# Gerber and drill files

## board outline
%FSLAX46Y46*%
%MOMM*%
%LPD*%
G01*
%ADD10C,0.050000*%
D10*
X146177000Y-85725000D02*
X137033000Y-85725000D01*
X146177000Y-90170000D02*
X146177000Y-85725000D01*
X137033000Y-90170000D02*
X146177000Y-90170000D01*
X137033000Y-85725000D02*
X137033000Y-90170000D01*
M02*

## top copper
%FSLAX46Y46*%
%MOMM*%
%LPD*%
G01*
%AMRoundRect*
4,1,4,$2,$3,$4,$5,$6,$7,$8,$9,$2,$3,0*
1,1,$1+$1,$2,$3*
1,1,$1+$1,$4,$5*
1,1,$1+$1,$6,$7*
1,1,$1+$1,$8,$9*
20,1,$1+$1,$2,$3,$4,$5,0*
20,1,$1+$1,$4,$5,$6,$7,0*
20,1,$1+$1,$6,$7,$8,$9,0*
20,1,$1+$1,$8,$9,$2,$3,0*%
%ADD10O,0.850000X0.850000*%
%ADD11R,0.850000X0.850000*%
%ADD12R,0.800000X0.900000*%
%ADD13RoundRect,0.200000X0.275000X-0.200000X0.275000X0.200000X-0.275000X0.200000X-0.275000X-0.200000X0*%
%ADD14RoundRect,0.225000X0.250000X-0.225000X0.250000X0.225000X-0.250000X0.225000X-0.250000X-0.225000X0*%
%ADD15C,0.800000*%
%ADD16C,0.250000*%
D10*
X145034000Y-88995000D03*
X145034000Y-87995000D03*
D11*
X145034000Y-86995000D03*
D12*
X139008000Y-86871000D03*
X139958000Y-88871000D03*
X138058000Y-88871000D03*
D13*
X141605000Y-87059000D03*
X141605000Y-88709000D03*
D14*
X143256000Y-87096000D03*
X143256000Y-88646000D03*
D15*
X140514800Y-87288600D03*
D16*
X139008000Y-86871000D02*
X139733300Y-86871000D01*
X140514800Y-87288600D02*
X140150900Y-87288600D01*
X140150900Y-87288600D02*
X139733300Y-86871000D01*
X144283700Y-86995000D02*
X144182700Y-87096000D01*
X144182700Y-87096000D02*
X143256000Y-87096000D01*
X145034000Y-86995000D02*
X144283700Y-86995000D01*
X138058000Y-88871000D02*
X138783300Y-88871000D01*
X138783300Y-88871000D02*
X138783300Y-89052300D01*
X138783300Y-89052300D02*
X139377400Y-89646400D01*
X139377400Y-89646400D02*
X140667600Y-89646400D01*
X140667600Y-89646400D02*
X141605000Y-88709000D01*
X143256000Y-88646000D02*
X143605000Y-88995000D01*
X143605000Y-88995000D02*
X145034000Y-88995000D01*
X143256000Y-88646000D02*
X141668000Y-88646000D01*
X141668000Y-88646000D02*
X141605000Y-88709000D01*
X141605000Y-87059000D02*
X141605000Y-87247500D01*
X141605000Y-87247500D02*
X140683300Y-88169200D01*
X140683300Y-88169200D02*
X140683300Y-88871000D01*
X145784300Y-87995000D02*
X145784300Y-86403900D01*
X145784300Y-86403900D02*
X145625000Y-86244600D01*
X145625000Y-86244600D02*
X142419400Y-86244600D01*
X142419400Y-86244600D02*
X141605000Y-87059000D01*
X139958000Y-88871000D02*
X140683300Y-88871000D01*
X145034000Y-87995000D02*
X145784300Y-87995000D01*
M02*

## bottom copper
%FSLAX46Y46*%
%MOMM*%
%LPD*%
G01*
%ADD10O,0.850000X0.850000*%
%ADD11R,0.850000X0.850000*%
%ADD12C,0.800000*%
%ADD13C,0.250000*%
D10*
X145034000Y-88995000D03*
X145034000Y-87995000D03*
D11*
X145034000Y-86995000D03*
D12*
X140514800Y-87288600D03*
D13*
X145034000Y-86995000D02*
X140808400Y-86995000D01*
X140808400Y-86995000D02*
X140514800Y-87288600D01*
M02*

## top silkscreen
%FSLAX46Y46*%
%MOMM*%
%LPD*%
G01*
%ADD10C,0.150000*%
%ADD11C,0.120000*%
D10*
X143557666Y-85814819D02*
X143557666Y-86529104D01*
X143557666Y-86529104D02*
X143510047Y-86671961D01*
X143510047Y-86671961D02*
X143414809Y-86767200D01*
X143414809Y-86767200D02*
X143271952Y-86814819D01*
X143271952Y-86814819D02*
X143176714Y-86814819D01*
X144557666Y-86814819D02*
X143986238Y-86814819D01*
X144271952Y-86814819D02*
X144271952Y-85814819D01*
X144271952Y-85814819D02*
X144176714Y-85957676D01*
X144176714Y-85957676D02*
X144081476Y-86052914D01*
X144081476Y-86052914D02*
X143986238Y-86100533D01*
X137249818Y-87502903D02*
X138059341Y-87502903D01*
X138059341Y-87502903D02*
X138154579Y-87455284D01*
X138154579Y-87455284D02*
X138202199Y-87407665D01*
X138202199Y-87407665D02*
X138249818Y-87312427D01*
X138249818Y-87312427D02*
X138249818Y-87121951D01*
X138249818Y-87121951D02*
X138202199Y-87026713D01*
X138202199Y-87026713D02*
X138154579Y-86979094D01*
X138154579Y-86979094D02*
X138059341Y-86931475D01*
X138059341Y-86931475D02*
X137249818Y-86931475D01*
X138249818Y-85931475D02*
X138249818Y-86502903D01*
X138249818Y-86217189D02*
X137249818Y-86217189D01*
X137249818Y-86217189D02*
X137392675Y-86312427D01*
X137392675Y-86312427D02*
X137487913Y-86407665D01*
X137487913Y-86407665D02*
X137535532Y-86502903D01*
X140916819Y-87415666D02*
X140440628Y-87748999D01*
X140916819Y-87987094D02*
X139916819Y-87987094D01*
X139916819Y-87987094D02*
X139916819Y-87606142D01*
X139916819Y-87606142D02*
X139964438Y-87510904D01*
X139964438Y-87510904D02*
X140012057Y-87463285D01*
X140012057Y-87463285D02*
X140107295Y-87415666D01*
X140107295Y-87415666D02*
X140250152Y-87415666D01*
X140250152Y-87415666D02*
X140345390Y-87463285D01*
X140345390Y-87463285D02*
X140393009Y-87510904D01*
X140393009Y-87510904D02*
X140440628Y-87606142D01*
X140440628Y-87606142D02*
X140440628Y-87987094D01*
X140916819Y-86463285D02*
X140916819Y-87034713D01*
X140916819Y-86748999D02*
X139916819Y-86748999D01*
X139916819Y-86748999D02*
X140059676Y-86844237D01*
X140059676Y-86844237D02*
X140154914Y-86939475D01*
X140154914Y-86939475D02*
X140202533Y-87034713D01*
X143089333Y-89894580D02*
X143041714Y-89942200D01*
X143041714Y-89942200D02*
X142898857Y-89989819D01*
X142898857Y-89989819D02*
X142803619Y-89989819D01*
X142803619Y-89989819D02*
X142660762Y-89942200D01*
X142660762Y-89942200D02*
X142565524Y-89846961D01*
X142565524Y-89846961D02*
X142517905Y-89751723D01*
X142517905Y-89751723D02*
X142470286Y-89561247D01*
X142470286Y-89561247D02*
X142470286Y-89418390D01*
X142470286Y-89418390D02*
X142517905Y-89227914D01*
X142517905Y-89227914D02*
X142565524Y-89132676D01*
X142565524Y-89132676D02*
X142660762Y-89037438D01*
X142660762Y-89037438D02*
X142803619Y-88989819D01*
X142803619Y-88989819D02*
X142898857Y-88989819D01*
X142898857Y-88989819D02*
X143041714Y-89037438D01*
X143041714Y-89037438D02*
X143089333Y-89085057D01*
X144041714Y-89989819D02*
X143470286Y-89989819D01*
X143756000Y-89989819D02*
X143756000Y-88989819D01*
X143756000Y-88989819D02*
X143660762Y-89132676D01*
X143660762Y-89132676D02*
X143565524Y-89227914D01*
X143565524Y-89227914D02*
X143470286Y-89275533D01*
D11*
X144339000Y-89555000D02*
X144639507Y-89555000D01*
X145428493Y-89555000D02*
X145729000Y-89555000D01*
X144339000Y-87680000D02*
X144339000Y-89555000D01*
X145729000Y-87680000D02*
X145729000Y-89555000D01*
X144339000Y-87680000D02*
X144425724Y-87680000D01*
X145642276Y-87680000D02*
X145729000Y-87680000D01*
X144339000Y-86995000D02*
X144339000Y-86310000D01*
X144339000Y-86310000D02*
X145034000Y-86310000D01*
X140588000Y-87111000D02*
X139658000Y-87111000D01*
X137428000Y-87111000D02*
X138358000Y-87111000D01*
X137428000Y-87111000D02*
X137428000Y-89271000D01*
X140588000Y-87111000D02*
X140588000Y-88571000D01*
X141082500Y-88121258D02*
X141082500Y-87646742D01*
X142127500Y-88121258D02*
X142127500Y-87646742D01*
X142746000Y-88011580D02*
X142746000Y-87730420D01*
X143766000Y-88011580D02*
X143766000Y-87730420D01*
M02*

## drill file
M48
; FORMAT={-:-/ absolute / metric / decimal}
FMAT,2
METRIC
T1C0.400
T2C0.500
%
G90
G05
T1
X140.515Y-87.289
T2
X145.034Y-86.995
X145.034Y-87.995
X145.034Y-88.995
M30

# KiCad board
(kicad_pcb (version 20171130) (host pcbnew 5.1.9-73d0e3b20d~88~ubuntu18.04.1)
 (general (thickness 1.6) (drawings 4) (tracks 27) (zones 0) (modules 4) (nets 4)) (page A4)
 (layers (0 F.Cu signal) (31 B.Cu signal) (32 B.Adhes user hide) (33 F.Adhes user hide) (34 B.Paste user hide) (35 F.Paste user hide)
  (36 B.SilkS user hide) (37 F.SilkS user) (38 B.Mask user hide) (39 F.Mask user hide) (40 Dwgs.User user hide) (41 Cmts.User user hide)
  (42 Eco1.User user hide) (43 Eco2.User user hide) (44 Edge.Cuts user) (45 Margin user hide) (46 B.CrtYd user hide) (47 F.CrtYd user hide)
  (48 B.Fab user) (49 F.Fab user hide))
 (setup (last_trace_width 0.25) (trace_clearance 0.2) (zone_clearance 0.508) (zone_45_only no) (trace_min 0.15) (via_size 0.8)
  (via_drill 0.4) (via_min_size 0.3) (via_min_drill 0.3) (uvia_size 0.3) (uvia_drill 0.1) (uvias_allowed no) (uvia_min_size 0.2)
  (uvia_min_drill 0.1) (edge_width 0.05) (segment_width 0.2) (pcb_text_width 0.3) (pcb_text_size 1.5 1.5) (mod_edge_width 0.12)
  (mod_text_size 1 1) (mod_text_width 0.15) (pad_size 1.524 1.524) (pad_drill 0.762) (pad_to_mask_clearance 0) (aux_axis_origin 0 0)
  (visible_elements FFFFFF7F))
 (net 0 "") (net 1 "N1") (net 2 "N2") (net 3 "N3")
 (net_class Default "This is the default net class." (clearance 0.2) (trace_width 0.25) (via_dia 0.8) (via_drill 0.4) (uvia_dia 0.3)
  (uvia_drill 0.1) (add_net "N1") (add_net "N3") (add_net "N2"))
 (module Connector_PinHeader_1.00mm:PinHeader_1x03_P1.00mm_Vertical (layer F.Cu) (at 145.034 86.995)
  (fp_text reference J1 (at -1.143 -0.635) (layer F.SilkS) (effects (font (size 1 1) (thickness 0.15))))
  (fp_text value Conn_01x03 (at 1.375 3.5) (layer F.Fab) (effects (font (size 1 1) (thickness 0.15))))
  (fp_line (start -0.695 2.56) (end -0.394493 2.56) (layer F.SilkS) (width 0.12))
  (fp_line (start 0.394493 2.56) (end 0.695 2.56) (layer F.SilkS) (width 0.12))
  (fp_line (start -0.695 0.685) (end -0.695 2.56) (layer F.SilkS) (width 0.12))
  (fp_line (start 0.695 0.685) (end 0.695 2.56) (layer F.SilkS) (width 0.12))
  (fp_line (start -0.695 0.685) (end -0.608276 0.685) (layer F.SilkS) (width 0.12))
  (fp_line (start 0.608276 0.685) (end 0.695 0.685) (layer F.SilkS) (width 0.12))
  (fp_line (start -0.695 0) (end -0.695 -0.685) (layer F.SilkS) (width 0.12))
  (fp_line (start -0.695 -0.685) (end 0 -0.685) (layer F.SilkS) (width 0.12))
  (pad 3 thru_hole oval (at 0 2) (size 0.85 0.85) (drill 0.5) (layers *.Cu *.Mask) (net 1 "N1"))
  (pad 2 thru_hole oval (at 0 1) (size 0.85 0.85) (drill 0.5) (layers *.Cu *.Mask) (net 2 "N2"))
  (pad 1 thru_hole rect (at 0 0) (size 0.85 0.85) (drill 0.5) (layers *.Cu *.Mask) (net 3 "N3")))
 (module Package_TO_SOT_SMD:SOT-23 (layer F.Cu) (at 139.008 87.871 90)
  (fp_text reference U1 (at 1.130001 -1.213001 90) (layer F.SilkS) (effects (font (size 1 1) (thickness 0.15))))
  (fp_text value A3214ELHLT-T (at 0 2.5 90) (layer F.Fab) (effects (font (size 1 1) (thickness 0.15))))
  (fp_line (start 0.76 1.58) (end 0.76 0.65) (layer F.SilkS) (width 0.12))
  (fp_line (start 0.76 -1.58) (end 0.76 -0.65) (layer F.SilkS) (width 0.12))
  (fp_line (start 0.76 -1.58) (end -1.4 -1.58) (layer F.SilkS) (width 0.12))
  (fp_line (start 0.76 1.58) (end -0.7 1.58) (layer F.SilkS) (width 0.12))
  (pad 3 smd rect (at 1 0 90) (size 0.9 0.8) (layers F.Cu F.Paste F.Mask) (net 3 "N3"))
  (pad 2 smd rect (at -1 0.95 90) (size 0.9 0.8) (layers F.Cu F.Paste F.Mask) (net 2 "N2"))
  (pad 1 smd rect (at -1 -0.95 90) (size 0.9 0.8) (layers F.Cu F.Paste F.Mask) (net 1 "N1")))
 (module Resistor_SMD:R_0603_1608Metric (layer F.Cu) (at 141.605 87.884 90)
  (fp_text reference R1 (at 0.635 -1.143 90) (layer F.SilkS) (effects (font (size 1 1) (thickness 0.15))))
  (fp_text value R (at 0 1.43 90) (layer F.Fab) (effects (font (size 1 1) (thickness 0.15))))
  (fp_line (start -0.237258 -0.5225) (end 0.237258 -0.5225) (layer F.SilkS) (width 0.12))
  (fp_line (start -0.237258 0.5225) (end 0.237258 0.5225) (layer F.SilkS) (width 0.12))
  (pad 2 smd roundrect (at 0.825 0 90) (size 0.8 0.95) (layers F.Cu F.Paste F.Mask) (roundrect_rratio 0.25) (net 2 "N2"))
  (pad 1 smd roundrect (at -0.825 0 90) (size 0.8 0.95) (layers F.Cu F.Paste F.Mask) (roundrect_rratio 0.25) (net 1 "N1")))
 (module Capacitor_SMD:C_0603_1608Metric (layer F.Cu) (at 143.256 87.871 90)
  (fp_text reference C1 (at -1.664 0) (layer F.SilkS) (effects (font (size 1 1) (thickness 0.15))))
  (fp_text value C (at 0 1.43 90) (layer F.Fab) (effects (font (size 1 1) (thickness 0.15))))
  (fp_line (start -0.14058 -0.51) (end 0.14058 -0.51) (layer F.SilkS) (width 0.12))
  (fp_line (start -0.14058 0.51) (end 0.14058 0.51) (layer F.SilkS) (width 0.12))
  (pad 2 smd roundrect (at 0.775 0 90) (size 0.9 0.95) (layers F.Cu F.Paste F.Mask) (roundrect_rratio 0.25) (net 3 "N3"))
  (pad 1 smd roundrect (at -0.775 0 90) (size 0.9 0.95) (layers F.Cu F.Paste F.Mask) (roundrect_rratio 0.25) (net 1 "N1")))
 (gr_line (start 146.177 85.725) (end 137.033 85.725) (layer Edge.Cuts) (width 0.05))
 (gr_line (start 146.177 90.17) (end 146.177 85.725) (layer Edge.Cuts) (width 0.05))
 (gr_line (start 137.033 90.17) (end 146.177 90.17) (layer Edge.Cuts) (width 0.05))
 (gr_line (start 137.033 85.725) (end 137.033 90.17) (layer Edge.Cuts) (width 0.05))
 (segment (start 139.008 86.871) (end 139.7333 86.871) (width 0.25) (layer F.Cu) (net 3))
 (segment (start 140.5148 87.2886) (end 140.1509 87.2886) (width 0.25) (layer F.Cu) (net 3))
 (segment (start 140.1509 87.2886) (end 139.7333 86.871) (width 0.25) (layer F.Cu) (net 3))
 (segment (start 145.034 86.995) (end 140.8084 86.995) (width 0.25) (layer B.Cu) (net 3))
 (segment (start 140.8084 86.995) (end 140.5148 87.2886) (width 0.25) (layer B.Cu) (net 3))
 (segment (start 144.2837 86.995) (end 144.1827 87.096) (width 0.25) (layer F.Cu) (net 3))
 (segment (start 144.1827 87.096) (end 143.256 87.096) (width 0.25) (layer F.Cu) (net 3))
 (segment (start 145.034 86.995) (end 144.2837 86.995) (width 0.25) (layer F.Cu) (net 3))
 (via (at 140.5148 87.2886) (size 0.8) (layers F.Cu B.Cu) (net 3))
 (segment (start 138.058 88.871) (end 138.7833 88.871) (width 0.25) (layer F.Cu) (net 1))
 (segment (start 138.7833 88.871) (end 138.7833 89.0523) (width 0.25) (layer F.Cu) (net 1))
 (segment (start 138.7833 89.0523) (end 139.3774 89.6464) (width 0.25) (layer F.Cu) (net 1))
 (segment (start 139.3774 89.6464) (end 140.6676 89.6464) (width 0.25) (layer F.Cu) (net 1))
 (segment (start 140.6676 89.6464) (end 141.605 88.709) (width 0.25) (layer F.Cu) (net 1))
 (segment (start 143.256 88.646) (end 143.605 88.995) (width 0.25) (layer F.Cu) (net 1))
 (segment (start 143.605 88.995) (end 145.034 88.995) (width 0.25) (layer F.Cu) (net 1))
 (segment (start 143.256 88.646) (end 141.668 88.646) (width 0.25) (layer F.Cu) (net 1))
 (segment (start 141.668 88.646) (end 141.605 88.709) (width 0.25) (layer F.Cu) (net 1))
 (segment (start 141.605 87.059) (end 141.605 87.2475) (width 0.25) (layer F.Cu) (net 2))
 (segment (start 141.605 87.2475) (end 140.6833 88.1692) (width 0.25) (layer F.Cu) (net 2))
 (segment (start 140.6833 88.1692) (end 140.6833 88.871) (width 0.25) (layer F.Cu) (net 2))
 (segment (start 145.7843 87.995) (end 145.7843 86.4039) (width 0.25) (layer F.Cu) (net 2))
 (segment (start 145.7843 86.4039) (end 145.625 86.2446) (width 0.25) (layer F.Cu) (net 2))
 (segment (start 145.625 86.2446) (end 142.4194 86.2446) (width 0.25) (layer F.Cu) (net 2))
 (segment (start 142.4194 86.2446) (end 141.605 87.059) (width 0.25) (layer F.Cu) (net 2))
 (segment (start 139.958 88.871) (end 140.6833 88.871) (width 0.25) (layer F.Cu) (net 2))
 (segment (start 145.034 87.995) (end 145.7843 87.995) (width 0.25) (layer F.Cu) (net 2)))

